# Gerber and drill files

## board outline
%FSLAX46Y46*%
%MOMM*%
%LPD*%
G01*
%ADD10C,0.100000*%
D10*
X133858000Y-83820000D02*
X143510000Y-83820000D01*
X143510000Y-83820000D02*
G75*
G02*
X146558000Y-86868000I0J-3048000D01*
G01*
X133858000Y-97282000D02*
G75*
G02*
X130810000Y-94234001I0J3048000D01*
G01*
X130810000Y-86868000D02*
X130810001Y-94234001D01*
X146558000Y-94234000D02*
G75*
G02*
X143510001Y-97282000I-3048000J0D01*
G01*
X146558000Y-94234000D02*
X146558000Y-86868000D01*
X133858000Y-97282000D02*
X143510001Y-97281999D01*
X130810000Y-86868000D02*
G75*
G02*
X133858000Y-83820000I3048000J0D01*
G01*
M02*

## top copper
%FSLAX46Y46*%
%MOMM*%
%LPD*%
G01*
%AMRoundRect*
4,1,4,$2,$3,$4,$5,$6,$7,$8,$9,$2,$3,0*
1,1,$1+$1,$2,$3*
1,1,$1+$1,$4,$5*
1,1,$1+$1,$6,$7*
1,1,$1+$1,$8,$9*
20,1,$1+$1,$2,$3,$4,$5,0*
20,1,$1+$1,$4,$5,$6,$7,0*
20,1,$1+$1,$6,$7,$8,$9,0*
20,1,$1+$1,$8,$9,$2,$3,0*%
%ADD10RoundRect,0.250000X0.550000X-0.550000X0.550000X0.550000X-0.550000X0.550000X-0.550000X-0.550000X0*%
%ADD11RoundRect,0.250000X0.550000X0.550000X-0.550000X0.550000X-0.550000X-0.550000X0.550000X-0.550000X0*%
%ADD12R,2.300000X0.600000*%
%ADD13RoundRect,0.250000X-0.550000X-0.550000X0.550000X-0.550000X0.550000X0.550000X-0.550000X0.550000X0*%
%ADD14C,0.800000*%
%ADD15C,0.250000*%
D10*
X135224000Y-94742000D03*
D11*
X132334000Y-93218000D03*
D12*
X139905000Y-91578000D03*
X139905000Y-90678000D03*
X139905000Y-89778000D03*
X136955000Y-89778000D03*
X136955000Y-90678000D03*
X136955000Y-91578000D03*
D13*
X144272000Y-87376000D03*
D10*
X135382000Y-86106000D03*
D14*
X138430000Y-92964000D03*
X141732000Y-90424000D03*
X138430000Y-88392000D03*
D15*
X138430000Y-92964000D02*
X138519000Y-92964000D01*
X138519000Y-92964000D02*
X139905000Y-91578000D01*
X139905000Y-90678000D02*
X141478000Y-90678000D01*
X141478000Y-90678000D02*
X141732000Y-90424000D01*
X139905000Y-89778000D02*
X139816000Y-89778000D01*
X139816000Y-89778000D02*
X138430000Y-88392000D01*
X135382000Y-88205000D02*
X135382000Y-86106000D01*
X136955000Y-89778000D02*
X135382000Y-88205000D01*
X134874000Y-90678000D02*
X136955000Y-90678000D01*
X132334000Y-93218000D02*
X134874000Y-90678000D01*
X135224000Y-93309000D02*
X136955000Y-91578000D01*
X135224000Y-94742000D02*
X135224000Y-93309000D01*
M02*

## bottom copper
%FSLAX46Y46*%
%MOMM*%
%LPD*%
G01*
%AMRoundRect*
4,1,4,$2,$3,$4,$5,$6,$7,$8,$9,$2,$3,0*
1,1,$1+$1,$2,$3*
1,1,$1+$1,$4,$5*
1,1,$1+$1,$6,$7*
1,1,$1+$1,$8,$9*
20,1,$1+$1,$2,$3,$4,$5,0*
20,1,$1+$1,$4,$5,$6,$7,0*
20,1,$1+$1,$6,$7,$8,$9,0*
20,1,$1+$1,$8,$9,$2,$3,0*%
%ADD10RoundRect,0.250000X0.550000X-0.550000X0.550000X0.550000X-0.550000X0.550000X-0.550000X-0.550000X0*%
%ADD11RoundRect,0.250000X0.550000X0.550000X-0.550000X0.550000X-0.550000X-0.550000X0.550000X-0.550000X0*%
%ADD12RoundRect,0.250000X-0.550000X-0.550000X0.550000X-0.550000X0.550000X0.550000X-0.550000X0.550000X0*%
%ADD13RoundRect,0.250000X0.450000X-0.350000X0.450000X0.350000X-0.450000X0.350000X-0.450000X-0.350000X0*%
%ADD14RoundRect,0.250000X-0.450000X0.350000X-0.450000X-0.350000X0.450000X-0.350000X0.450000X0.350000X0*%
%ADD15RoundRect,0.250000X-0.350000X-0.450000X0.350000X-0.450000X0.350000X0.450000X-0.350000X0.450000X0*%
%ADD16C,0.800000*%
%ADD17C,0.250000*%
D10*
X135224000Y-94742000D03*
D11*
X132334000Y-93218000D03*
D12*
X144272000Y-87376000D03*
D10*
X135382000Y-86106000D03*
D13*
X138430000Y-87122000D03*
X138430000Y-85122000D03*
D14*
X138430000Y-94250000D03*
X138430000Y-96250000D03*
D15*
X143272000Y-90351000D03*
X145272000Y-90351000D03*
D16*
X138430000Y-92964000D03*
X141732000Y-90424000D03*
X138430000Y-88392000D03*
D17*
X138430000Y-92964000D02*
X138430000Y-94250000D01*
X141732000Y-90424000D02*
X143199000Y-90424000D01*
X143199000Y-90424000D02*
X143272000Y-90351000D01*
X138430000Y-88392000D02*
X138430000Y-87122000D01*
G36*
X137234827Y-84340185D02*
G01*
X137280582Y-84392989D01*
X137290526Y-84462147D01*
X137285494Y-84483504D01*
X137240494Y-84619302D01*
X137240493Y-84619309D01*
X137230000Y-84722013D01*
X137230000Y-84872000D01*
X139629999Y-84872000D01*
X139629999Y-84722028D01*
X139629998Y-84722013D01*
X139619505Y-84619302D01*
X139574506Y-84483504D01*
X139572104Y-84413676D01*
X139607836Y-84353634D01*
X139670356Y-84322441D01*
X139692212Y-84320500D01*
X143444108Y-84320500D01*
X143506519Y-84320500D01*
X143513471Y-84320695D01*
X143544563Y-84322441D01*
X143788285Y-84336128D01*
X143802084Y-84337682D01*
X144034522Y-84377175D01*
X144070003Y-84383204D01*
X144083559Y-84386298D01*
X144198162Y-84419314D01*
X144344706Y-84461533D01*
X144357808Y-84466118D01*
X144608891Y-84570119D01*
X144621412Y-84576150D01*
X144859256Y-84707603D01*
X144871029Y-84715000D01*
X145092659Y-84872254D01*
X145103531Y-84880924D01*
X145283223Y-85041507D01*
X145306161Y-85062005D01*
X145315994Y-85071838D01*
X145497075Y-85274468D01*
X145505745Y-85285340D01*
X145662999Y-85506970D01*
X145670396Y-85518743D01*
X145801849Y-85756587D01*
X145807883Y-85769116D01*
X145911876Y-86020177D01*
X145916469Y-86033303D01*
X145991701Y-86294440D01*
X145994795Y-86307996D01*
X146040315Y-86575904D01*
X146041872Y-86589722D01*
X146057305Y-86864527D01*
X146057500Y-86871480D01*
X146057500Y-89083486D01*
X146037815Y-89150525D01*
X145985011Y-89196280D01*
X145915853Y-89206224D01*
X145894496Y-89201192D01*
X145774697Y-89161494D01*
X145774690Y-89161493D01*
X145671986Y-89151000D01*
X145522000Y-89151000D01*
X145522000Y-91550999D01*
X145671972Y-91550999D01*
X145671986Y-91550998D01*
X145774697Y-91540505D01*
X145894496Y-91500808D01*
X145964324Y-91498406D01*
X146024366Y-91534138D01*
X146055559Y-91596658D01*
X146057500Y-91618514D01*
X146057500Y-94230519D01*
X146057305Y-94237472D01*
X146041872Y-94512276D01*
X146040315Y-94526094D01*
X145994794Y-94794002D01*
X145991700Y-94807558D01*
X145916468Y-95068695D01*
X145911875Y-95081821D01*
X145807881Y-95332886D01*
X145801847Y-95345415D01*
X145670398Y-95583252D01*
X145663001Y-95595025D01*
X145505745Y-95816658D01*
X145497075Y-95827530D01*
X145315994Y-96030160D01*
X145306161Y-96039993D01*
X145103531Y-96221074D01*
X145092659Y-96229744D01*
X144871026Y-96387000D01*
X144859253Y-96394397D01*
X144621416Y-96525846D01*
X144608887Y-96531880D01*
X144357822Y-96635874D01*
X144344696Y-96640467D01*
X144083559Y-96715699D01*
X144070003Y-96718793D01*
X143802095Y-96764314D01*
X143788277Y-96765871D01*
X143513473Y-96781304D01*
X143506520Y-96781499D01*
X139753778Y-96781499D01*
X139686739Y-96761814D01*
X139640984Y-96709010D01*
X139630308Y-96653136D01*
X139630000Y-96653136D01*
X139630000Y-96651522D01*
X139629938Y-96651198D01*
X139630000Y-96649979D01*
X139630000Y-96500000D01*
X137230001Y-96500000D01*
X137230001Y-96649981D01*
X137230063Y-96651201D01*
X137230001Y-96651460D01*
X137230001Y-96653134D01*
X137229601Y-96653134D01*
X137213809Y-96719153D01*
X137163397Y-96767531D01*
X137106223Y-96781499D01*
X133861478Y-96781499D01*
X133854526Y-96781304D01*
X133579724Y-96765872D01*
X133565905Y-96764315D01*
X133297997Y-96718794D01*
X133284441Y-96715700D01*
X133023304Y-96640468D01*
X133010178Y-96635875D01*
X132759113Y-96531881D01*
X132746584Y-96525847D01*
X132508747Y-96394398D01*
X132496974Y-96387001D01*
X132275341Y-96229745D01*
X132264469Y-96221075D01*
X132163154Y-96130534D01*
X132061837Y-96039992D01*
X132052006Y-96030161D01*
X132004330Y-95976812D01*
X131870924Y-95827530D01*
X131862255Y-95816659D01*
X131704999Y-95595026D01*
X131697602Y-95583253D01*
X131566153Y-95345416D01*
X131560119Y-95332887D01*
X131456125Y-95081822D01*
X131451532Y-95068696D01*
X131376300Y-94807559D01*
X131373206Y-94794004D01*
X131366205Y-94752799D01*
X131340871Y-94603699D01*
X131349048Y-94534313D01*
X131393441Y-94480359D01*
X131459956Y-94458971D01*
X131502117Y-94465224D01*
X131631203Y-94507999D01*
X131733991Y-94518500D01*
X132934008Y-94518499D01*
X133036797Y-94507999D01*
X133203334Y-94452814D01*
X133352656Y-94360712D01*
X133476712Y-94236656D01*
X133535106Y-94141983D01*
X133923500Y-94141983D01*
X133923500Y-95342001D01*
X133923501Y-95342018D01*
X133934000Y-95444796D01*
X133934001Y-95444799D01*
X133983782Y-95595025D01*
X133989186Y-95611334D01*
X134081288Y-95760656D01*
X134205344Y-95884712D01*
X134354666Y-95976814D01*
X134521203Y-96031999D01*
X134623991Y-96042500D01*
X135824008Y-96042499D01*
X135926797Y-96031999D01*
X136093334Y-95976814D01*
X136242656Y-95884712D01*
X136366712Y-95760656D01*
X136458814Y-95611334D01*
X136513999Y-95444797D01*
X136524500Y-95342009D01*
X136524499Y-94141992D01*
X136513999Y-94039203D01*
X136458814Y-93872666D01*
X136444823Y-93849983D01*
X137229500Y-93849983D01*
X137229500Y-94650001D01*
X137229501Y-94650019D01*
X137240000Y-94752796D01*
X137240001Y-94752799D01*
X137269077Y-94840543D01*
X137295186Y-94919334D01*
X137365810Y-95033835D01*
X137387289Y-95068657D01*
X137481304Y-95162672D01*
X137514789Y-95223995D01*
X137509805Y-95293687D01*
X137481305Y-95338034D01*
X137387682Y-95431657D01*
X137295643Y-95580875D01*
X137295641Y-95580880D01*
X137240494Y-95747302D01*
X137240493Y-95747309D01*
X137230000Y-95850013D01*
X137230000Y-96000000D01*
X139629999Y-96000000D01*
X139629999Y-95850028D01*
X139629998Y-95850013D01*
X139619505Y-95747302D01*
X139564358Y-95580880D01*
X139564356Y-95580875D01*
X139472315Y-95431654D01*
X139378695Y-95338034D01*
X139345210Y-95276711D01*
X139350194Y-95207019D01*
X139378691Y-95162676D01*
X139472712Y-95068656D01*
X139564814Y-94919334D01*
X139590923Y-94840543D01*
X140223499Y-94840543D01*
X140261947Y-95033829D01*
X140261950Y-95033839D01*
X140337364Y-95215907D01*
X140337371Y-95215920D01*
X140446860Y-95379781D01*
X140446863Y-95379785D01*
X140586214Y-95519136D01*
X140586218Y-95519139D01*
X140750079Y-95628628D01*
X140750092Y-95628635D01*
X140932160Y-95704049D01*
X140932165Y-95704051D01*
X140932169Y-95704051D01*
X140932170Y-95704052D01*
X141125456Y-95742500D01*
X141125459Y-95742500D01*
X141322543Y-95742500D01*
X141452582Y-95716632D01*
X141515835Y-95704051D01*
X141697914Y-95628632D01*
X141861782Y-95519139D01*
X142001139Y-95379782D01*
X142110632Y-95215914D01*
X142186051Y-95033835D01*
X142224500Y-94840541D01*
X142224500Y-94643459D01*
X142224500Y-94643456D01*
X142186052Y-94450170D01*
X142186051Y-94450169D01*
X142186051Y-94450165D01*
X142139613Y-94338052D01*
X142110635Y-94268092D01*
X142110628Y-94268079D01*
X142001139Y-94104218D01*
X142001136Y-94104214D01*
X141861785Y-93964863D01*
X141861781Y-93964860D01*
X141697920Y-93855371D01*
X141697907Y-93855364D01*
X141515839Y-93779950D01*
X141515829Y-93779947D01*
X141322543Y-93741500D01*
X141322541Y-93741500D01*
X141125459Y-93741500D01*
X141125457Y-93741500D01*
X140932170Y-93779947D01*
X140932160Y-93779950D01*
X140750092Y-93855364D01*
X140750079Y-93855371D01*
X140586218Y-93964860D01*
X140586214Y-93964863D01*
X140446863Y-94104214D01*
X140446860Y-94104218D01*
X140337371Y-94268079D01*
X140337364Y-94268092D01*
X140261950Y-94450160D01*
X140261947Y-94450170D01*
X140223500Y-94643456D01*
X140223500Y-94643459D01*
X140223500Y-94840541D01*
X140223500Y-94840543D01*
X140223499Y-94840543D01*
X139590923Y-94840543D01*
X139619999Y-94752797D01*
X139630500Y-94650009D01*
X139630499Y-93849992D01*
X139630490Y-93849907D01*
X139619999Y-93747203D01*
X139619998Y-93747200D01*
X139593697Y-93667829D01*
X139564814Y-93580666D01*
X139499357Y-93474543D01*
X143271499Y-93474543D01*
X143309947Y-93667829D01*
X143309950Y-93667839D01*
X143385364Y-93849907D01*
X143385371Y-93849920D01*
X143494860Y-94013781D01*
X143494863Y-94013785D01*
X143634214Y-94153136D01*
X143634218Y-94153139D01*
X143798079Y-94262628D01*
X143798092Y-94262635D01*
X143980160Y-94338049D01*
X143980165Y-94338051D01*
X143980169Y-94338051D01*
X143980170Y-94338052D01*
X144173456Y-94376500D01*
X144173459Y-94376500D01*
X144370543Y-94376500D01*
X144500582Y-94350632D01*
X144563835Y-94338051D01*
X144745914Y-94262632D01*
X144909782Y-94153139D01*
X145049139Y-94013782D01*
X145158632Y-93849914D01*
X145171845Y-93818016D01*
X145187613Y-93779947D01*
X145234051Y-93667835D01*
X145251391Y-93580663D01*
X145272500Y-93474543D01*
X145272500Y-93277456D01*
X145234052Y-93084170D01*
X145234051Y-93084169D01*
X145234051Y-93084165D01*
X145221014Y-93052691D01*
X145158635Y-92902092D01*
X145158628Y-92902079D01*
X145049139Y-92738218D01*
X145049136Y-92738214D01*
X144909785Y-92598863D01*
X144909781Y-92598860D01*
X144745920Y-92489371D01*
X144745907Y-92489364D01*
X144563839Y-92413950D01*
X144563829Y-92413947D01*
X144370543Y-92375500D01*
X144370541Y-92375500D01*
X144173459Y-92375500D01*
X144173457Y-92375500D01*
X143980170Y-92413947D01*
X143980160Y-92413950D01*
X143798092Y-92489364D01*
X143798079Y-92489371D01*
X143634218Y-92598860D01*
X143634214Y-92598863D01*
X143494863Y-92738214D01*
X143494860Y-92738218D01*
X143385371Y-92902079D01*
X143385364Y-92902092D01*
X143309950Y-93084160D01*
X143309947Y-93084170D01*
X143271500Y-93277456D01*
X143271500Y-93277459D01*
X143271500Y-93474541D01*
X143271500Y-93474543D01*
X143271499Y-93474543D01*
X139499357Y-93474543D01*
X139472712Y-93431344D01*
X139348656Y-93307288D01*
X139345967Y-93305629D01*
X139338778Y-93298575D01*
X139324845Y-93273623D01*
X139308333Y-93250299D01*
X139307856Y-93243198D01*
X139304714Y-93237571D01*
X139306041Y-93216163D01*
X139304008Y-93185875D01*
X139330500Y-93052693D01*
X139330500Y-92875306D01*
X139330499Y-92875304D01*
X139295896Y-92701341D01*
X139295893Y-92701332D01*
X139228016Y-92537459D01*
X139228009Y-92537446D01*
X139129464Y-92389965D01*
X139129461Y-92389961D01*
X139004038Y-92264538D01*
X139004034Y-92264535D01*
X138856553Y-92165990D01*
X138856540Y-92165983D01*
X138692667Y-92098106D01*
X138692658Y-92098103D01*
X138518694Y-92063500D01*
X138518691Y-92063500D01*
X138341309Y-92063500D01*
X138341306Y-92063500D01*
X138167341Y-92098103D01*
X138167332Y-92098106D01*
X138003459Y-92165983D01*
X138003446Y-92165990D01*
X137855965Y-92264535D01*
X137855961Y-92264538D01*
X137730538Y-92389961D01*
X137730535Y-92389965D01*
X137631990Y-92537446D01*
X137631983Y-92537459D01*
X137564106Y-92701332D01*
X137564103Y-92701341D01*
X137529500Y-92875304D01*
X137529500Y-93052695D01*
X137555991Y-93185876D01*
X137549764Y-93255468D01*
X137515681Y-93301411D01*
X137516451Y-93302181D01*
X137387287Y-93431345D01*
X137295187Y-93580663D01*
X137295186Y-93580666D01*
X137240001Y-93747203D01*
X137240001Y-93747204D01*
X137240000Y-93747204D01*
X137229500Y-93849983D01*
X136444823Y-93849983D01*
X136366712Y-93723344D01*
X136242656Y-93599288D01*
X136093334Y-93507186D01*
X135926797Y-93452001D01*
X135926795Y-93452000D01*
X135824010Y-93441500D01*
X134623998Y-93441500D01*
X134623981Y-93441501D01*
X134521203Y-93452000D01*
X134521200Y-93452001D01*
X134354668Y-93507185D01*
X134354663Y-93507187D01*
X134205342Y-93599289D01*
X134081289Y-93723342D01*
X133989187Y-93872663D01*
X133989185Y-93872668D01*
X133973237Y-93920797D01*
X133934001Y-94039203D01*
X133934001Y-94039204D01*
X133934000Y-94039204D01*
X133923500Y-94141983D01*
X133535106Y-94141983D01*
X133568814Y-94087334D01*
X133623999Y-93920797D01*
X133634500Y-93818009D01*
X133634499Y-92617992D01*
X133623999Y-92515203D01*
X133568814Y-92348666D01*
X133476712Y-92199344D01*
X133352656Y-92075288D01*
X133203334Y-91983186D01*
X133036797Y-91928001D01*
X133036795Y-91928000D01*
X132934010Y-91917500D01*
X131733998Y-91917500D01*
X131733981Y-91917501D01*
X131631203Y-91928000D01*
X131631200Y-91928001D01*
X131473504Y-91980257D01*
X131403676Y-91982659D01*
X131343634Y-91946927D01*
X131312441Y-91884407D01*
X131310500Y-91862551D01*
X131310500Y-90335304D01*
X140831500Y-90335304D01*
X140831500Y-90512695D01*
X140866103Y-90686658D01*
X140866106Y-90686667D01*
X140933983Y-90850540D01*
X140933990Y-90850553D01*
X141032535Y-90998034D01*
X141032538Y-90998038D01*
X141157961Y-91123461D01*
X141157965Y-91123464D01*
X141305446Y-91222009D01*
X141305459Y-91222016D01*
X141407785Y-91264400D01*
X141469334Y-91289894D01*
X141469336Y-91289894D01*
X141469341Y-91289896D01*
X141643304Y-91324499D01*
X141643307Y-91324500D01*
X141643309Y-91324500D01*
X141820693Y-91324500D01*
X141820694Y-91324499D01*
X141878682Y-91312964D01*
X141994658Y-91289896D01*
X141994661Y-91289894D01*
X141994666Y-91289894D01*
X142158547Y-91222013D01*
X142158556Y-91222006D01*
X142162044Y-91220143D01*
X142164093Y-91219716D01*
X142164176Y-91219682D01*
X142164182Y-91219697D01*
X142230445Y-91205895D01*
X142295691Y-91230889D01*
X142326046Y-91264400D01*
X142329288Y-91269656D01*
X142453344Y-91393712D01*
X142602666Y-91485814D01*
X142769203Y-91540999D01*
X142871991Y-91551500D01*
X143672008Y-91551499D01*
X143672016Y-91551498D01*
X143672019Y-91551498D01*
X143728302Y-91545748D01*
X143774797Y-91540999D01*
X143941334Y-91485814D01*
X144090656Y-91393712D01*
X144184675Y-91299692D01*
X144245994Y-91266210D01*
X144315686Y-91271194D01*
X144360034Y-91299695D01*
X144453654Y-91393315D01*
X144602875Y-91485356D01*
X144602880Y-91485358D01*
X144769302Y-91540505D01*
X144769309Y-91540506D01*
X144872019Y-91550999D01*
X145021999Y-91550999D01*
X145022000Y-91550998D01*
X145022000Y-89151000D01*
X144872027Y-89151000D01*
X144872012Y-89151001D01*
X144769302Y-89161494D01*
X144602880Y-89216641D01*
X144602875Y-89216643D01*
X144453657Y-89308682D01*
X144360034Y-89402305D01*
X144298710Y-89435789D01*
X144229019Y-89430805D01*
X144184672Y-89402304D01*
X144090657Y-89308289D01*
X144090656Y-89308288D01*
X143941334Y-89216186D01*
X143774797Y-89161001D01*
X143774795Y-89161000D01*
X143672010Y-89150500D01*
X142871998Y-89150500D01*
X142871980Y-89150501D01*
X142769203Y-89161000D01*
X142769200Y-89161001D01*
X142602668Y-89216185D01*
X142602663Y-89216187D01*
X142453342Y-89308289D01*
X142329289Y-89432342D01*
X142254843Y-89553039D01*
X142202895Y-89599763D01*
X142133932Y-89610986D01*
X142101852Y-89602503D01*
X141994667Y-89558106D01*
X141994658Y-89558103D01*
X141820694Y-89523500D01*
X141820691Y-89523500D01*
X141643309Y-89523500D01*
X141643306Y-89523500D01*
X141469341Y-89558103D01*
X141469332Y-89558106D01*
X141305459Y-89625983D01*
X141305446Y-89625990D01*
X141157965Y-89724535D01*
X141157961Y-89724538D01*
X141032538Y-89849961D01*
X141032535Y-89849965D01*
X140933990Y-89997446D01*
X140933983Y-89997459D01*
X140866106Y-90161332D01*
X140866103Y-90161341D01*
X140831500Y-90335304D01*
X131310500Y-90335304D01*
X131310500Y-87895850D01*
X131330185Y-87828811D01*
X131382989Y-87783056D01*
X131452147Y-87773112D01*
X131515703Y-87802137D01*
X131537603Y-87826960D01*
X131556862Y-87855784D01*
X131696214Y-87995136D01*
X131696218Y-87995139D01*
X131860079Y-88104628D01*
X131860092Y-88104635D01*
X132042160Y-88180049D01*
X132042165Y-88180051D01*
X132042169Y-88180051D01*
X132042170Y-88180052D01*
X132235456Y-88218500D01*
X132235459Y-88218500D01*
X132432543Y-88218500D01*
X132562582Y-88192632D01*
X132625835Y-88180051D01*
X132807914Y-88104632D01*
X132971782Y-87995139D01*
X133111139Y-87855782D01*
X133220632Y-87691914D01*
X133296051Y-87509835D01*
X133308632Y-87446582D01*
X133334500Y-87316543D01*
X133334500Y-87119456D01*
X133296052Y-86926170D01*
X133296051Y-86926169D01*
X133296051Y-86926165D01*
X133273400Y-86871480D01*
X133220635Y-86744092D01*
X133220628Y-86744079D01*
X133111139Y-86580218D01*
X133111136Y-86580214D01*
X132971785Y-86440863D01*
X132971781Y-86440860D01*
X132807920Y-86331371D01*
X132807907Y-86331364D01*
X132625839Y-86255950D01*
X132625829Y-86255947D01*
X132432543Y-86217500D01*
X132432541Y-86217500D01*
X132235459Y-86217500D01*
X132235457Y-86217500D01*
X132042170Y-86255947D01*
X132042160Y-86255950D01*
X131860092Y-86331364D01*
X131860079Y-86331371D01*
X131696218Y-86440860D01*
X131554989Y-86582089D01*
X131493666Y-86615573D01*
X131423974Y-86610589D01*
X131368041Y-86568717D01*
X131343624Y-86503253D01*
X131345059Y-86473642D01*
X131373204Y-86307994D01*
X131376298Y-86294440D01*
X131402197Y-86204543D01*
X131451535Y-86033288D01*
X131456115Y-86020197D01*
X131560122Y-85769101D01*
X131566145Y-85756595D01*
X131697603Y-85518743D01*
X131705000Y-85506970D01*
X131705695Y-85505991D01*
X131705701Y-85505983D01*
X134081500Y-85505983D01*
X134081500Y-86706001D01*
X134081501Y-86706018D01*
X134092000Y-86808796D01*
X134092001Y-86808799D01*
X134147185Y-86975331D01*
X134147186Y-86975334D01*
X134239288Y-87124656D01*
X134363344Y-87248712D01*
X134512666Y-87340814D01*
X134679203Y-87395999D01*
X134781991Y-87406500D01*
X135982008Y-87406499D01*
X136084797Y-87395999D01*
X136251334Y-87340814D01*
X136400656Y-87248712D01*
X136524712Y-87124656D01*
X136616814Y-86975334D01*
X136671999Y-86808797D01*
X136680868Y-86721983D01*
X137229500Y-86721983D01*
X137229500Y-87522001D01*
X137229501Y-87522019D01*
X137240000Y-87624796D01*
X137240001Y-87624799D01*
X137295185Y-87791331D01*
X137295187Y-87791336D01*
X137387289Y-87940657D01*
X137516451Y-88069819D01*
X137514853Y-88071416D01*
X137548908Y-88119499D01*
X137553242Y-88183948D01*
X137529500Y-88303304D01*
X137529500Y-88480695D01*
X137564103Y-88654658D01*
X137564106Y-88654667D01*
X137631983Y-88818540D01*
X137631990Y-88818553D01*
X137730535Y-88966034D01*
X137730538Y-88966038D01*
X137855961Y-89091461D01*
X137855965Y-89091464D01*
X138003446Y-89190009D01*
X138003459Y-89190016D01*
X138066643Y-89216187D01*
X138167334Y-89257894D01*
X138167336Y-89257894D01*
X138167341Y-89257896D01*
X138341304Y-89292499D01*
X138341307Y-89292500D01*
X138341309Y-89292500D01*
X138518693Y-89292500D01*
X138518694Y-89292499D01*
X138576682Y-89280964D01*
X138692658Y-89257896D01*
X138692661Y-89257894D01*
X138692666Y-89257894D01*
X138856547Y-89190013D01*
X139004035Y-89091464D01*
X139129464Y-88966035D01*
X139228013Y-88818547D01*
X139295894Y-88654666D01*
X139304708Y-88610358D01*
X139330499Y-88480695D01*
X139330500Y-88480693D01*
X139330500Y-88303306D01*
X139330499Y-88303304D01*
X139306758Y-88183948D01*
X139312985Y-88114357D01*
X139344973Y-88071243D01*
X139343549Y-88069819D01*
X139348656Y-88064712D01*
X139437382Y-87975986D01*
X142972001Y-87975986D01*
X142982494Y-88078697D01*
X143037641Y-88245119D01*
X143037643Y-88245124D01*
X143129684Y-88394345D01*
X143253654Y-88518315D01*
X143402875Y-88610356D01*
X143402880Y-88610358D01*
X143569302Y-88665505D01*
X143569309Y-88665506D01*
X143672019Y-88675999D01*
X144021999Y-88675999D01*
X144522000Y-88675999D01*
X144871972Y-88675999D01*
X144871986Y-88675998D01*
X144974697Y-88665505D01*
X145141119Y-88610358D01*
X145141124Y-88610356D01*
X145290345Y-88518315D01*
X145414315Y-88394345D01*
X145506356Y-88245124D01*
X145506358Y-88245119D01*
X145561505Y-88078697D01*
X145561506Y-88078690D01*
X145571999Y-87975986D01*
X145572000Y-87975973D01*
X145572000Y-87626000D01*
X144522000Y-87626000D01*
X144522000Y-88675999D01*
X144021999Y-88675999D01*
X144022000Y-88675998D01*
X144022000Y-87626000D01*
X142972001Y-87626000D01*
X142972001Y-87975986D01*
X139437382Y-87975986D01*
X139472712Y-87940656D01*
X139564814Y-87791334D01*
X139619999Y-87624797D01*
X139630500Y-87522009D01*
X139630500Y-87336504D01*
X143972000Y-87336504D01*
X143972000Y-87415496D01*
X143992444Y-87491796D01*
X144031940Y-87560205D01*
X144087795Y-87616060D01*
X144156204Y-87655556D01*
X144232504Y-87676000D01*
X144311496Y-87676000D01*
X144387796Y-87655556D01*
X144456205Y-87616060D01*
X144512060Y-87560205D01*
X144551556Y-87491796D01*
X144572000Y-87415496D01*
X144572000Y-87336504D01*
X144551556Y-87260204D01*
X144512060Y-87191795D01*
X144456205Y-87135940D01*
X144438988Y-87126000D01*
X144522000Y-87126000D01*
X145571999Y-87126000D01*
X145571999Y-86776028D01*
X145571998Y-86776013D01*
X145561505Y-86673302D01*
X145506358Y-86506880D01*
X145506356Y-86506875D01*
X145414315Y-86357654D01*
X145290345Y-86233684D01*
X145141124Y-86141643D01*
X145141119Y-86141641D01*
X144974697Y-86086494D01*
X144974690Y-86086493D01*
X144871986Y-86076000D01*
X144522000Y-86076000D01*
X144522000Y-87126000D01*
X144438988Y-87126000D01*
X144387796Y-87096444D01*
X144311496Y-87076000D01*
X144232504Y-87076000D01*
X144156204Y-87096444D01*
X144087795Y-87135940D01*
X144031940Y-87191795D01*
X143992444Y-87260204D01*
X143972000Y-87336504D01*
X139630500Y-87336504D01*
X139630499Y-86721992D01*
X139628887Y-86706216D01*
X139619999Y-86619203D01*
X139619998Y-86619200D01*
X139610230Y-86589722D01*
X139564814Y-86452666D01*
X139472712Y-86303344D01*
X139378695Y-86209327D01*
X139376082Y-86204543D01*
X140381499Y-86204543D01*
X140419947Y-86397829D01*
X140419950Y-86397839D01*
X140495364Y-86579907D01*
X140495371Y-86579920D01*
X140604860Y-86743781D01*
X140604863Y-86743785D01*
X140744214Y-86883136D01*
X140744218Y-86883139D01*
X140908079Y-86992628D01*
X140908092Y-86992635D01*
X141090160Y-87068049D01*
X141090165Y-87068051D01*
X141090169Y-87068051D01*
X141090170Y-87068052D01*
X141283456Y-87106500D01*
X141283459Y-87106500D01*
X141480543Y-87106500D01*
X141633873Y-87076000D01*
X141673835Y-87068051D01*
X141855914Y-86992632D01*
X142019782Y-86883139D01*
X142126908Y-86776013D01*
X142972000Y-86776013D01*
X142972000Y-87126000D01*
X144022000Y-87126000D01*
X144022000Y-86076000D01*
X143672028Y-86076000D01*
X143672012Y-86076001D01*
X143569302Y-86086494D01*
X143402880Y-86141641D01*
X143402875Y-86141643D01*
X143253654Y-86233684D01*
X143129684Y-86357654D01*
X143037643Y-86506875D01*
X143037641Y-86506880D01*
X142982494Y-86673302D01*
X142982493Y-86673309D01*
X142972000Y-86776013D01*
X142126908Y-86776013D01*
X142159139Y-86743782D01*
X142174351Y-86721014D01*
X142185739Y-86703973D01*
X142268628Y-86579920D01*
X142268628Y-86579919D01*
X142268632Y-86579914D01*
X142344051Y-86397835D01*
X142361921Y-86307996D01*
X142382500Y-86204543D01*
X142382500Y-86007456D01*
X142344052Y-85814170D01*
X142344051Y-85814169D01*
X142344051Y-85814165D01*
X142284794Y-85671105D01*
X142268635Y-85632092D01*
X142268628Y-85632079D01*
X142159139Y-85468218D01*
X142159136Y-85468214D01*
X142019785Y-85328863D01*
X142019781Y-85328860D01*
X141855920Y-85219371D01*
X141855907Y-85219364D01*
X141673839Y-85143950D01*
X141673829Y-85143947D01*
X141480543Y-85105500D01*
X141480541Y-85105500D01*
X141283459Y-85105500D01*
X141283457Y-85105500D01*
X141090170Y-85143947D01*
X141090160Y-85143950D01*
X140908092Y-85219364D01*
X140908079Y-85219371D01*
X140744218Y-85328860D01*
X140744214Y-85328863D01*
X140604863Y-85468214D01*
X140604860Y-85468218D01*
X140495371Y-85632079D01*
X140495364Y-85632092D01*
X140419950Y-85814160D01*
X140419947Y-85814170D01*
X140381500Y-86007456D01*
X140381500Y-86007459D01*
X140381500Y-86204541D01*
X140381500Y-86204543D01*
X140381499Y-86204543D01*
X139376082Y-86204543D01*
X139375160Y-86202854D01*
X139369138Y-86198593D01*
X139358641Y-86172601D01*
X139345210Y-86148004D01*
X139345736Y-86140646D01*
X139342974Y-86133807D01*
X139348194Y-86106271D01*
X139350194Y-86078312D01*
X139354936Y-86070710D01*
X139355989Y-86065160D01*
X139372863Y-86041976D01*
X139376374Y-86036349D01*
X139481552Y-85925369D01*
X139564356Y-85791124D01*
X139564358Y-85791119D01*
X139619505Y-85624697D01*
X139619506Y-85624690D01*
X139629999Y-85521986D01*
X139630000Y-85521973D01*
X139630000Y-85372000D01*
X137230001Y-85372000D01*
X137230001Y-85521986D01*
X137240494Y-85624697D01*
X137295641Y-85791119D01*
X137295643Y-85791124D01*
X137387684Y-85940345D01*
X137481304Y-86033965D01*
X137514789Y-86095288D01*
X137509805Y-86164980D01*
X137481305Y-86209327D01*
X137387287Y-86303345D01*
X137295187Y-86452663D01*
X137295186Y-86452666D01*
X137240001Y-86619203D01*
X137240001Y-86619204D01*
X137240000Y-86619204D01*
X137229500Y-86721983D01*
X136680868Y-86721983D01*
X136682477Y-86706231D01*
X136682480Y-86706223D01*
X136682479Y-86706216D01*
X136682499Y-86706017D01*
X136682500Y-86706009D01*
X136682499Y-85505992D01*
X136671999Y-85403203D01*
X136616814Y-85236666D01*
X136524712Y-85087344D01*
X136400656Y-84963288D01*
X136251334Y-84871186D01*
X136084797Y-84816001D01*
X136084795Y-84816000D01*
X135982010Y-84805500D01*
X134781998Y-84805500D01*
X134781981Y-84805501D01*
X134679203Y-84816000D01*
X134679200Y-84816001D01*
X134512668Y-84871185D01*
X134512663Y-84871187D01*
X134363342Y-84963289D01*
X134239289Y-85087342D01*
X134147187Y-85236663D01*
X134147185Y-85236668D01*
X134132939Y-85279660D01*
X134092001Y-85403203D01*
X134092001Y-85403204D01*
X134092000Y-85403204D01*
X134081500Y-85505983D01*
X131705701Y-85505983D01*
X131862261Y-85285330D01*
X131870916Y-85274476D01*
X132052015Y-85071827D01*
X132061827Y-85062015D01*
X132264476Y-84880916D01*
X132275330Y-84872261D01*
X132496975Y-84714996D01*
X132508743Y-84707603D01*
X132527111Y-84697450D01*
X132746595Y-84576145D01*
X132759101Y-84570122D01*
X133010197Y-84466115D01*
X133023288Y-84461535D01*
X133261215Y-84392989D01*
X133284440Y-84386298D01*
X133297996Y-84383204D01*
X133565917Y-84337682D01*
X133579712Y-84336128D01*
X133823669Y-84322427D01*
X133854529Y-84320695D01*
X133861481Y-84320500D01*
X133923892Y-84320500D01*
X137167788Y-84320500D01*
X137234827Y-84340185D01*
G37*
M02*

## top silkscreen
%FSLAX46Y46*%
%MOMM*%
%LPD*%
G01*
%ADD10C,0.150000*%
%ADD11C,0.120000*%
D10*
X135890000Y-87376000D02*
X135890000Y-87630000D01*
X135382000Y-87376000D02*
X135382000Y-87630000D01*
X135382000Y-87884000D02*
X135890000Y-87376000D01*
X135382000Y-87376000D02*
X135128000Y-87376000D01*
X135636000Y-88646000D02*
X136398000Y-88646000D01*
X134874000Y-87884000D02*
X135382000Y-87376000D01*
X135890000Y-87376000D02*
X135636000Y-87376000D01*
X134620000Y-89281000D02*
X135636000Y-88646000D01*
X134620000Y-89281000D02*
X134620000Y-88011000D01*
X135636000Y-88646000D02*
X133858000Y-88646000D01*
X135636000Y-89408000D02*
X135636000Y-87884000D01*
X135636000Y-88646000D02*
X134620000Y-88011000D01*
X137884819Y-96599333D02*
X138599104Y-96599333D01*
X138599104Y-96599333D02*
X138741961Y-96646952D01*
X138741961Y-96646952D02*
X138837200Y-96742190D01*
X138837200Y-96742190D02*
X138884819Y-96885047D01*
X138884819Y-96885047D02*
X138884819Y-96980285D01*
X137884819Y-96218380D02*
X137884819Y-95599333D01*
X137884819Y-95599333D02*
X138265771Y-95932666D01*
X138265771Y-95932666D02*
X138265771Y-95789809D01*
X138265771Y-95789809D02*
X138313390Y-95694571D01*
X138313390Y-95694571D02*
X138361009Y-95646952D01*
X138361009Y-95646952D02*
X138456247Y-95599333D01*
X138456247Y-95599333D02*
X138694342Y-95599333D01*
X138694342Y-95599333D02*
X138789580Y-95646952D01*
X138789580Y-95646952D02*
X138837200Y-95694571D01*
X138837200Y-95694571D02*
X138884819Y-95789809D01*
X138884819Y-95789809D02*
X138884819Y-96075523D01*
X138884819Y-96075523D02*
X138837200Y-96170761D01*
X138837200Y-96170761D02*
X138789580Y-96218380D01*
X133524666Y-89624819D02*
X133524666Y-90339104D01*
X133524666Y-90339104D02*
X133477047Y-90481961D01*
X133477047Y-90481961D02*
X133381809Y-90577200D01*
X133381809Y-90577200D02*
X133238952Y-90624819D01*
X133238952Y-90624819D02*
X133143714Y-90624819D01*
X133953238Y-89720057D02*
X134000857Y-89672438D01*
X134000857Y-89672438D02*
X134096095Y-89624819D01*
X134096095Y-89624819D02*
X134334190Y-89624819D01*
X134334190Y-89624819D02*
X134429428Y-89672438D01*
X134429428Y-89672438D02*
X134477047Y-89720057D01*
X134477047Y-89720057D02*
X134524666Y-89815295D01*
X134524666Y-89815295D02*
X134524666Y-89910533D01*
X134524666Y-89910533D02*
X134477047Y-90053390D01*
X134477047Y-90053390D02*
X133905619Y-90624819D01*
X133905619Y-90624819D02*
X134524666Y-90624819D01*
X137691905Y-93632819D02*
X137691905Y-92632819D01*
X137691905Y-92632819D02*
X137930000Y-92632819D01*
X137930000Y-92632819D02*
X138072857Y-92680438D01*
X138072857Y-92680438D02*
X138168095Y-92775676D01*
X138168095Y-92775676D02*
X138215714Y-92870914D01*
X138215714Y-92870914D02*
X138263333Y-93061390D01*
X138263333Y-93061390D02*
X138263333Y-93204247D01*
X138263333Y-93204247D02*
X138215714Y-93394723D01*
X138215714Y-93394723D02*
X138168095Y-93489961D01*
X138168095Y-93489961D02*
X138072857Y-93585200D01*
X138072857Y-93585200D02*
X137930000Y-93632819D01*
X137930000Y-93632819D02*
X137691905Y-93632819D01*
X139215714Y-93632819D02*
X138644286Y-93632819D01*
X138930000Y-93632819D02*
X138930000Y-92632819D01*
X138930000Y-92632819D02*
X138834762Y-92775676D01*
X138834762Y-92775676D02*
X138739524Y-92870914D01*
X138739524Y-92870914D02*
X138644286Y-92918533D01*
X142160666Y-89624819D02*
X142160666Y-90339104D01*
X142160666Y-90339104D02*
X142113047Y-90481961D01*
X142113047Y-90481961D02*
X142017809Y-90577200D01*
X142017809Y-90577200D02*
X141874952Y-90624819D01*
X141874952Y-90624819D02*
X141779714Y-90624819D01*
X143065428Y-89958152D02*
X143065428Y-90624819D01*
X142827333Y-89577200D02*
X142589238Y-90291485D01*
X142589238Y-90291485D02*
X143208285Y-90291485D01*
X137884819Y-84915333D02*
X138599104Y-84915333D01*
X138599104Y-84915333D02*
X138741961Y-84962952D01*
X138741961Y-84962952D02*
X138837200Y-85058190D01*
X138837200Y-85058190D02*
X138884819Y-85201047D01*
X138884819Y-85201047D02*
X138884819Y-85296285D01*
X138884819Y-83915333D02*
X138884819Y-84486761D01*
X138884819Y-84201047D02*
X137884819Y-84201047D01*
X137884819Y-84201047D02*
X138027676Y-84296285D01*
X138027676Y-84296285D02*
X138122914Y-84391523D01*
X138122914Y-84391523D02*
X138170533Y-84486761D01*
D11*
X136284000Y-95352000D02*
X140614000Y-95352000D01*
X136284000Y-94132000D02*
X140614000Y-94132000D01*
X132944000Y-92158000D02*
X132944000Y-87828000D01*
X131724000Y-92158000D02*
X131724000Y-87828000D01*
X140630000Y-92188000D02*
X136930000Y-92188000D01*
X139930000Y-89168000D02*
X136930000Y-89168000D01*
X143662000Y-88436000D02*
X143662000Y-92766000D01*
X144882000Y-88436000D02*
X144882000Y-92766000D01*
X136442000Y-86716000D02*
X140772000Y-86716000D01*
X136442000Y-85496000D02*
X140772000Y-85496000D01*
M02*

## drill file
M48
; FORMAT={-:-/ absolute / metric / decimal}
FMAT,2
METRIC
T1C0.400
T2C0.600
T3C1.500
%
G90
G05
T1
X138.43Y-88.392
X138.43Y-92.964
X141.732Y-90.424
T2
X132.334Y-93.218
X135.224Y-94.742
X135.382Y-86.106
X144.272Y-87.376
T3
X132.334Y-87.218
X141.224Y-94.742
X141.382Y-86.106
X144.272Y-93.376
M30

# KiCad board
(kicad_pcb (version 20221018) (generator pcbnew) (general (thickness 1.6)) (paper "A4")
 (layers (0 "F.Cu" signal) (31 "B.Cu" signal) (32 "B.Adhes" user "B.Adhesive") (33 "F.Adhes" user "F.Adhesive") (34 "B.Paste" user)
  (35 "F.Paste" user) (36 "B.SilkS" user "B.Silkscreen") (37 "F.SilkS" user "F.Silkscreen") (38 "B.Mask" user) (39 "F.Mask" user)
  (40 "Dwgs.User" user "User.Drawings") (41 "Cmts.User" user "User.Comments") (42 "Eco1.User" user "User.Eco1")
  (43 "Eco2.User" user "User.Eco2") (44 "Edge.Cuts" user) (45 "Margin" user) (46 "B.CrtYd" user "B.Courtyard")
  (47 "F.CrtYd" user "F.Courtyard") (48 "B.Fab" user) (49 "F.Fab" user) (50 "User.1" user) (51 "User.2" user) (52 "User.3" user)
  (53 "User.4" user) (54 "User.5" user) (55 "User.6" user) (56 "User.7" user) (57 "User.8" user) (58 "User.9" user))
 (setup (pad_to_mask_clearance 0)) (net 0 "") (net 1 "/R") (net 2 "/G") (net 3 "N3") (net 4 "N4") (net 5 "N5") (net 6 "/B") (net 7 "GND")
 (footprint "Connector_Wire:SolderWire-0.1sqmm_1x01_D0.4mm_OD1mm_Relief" (layer "F.Cu") (at 135.224 94.742 90)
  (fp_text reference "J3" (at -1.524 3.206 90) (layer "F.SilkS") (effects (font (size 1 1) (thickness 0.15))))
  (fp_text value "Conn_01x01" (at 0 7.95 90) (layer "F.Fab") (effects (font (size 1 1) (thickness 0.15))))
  (fp_line (start -0.61 1.06) (end -0.61 5.39) (stroke (width 0.12) (type solid)) (layer "F.SilkS"))
  (fp_line (start 0.61 1.06) (end 0.61 5.39) (stroke (width 0.12) (type solid)) (layer "F.SilkS"))
  (pad "" np_thru_hole circle (at 0 6 90) (size 1.5 1.5) (drill 1.5) (layers "*.Cu" "*.Mask"))
  (pad "1" thru_hole roundrect (at 0 0 90) (size 1.6 1.6) (drill 0.6) (layers "*.Cu" "*.Mask") (roundrect_rratio 0.15625) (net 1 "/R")))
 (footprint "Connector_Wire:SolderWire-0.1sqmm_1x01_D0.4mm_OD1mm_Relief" (layer "F.Cu") (at 132.334 93.218 180)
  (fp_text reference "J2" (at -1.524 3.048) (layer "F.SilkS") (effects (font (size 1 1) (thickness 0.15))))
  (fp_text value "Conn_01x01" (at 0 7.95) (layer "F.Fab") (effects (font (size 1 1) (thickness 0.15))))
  (fp_line (start -0.61 1.06) (end -0.61 5.39) (stroke (width 0.12) (type solid)) (layer "F.SilkS"))
  (fp_line (start 0.61 1.06) (end 0.61 5.39) (stroke (width 0.12) (type solid)) (layer "F.SilkS"))
  (pad "" np_thru_hole circle (at 0 6 180) (size 1.5 1.5) (drill 1.5) (layers "*.Cu" "*.Mask"))
  (pad "1" thru_hole roundrect (at 0 0 180) (size 1.6 1.6) (drill 0.6) (layers "*.Cu" "*.Mask") (roundrect_rratio 0.15625) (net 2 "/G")))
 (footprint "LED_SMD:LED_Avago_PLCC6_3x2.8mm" (layer "F.Cu") (at 138.43 90.678 180)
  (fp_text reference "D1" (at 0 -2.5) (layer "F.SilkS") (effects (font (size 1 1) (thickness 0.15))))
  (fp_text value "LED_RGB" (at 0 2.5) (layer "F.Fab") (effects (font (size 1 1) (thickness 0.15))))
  (fp_line (start -2.2 -1.51) (end 1.5 -1.51) (stroke (width 0.12) (type solid)) (layer "F.SilkS"))
  (fp_line (start -1.5 1.51) (end 1.5 1.51) (stroke (width 0.12) (type solid)) (layer "F.SilkS"))
  (pad "1" smd rect (at -1.475 -0.9 180) (size 2.3 0.6) (layers "F.Cu" "F.Paste" "F.Mask") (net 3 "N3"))
  (pad "2" smd rect (at -1.475 0 180) (size 2.3 0.6) (layers "F.Cu" "F.Paste" "F.Mask") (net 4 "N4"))
  (pad "3" smd rect (at -1.475 0.9 180) (size 2.3 0.6) (layers "F.Cu" "F.Paste" "F.Mask") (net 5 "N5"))
  (pad "4" smd rect (at 1.475 0.9 180) (size 2.3 0.6) (layers "F.Cu" "F.Paste" "F.Mask") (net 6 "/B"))
  (pad "5" smd rect (at 1.475 0 180) (size 2.3 0.6) (layers "F.Cu" "F.Paste" "F.Mask") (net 2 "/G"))
  (pad "6" smd rect (at 1.475 -0.9 180) (size 2.3 0.6) (layers "F.Cu" "F.Paste" "F.Mask") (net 1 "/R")))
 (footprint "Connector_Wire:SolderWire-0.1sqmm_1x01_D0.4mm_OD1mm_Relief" (layer "F.Cu") (at 144.272 87.376)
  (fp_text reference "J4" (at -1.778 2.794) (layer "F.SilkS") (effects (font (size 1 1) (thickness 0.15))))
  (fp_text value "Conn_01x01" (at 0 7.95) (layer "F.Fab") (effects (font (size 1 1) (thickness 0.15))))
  (fp_line (start -0.61 1.06) (end -0.61 5.39) (stroke (width 0.12) (type solid)) (layer "F.SilkS"))
  (fp_line (start 0.61 1.06) (end 0.61 5.39) (stroke (width 0.12) (type solid)) (layer "F.SilkS"))
  (pad "" np_thru_hole circle (at 0 6) (size 1.5 1.5) (drill 1.5) (layers "*.Cu" "*.Mask"))
  (pad "1" thru_hole roundrect (at 0 0) (size 1.6 1.6) (drill 0.6) (layers "*.Cu" "*.Mask") (roundrect_rratio 0.15625) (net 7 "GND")))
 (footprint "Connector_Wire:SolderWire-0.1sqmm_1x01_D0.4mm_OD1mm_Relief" (layer "F.Cu") (at 135.382 86.106 90)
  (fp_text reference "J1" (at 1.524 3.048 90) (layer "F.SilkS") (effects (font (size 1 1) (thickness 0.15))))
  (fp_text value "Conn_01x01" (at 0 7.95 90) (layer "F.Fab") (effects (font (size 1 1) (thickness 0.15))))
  (fp_line (start -0.61 1.06) (end -0.61 5.39) (stroke (width 0.12) (type solid)) (layer "F.SilkS"))
  (fp_line (start 0.61 1.06) (end 0.61 5.39) (stroke (width 0.12) (type solid)) (layer "F.SilkS"))
  (pad "" np_thru_hole circle (at 0 6 90) (size 1.5 1.5) (drill 1.5) (layers "*.Cu" "*.Mask"))
  (pad "1" thru_hole roundrect (at 0 0 90) (size 1.6 1.6) (drill 0.6) (layers "*.Cu" "*.Mask") (roundrect_rratio 0.15625) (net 6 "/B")))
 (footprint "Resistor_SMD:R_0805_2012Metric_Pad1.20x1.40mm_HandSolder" (layer "B.Cu") (at 138.43 86.122 90)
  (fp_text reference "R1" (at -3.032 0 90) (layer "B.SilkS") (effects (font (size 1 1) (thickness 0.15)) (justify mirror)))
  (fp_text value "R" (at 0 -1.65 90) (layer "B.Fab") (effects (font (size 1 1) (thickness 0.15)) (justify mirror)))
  (pad "1" smd roundrect (at -1 0 90) (size 1.2 1.4) (layers "B.Cu" "B.Paste" "B.Mask") (roundrect_rratio 0.208333) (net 5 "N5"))
  (pad "2" smd roundrect (at 1 0 90) (size 1.2 1.4) (layers "B.Cu" "B.Paste" "B.Mask") (roundrect_rratio 0.208333) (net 7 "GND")))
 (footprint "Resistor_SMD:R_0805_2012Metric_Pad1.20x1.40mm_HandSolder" (layer "B.Cu") (at 138.43 95.25 -90)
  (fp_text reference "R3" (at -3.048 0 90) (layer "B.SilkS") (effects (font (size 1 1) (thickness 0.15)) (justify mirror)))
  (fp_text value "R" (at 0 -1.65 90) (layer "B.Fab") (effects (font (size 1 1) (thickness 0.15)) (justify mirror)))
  (pad "1" smd roundrect (at -1 0 270) (size 1.2 1.4) (layers "B.Cu" "B.Paste" "B.Mask") (roundrect_rratio 0.208333) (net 3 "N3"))
  (pad "2" smd roundrect (at 1 0 270) (size 1.2 1.4) (layers "B.Cu" "B.Paste" "B.Mask") (roundrect_rratio 0.208333) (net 7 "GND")))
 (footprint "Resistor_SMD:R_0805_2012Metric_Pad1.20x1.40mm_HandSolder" (layer "B.Cu") (at 144.272 90.351)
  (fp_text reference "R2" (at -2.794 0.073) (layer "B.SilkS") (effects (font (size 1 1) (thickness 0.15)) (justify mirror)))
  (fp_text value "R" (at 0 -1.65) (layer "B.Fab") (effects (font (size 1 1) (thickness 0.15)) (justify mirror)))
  (pad "1" smd roundrect (at -1 0) (size 1.2 1.4) (layers "B.Cu" "B.Paste" "B.Mask") (roundrect_rratio 0.208333) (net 4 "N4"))
  (pad "2" smd roundrect (at 1 0) (size 1.2 1.4) (layers "B.Cu" "B.Paste" "B.Mask") (roundrect_rratio 0.208333) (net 7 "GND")))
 (gr_line (start 135.89 87.376) (end 135.89 87.63) (stroke (width 0.15) (type default)) (layer "F.SilkS"))
 (gr_line (start 135.382 87.376) (end 135.382 87.63) (stroke (width 0.15) (type default)) (layer "F.SilkS"))
 (gr_line (start 135.382 87.884) (end 135.89 87.376) (stroke (width 0.15) (type default)) (layer "F.SilkS"))
 (gr_line (start 135.382 87.376) (end 135.128 87.376) (stroke (width 0.15) (type default)) (layer "F.SilkS"))
 (gr_line (start 135.636 88.646) (end 136.398 88.646) (stroke (width 0.15) (type default)) (layer "F.SilkS"))
 (gr_line (start 134.874 87.884) (end 135.382 87.376) (stroke (width 0.15) (type default)) (layer "F.SilkS"))
 (gr_line (start 135.89 87.376) (end 135.636 87.376) (stroke (width 0.15) (type default)) (layer "F.SilkS"))
 (gr_line (start 134.62 89.281) (end 135.636 88.646) (stroke (width 0.15) (type default)) (layer "F.SilkS"))
 (gr_line (start 134.62 89.281) (end 134.62 88.011) (stroke (width 0.15) (type default)) (layer "F.SilkS"))
 (gr_line (start 135.636 88.646) (end 133.858 88.646) (stroke (width 0.15) (type default)) (layer "F.SilkS"))
 (gr_line (start 135.636 89.408) (end 135.636 87.884) (stroke (width 0.15) (type default)) (layer "F.SilkS"))
 (gr_line (start 135.636 88.646) (end 134.62 88.011) (stroke (width 0.15) (type default)) (layer "F.SilkS"))
 (gr_line (start 133.858 83.82) (end 143.51 83.82) (stroke (width 0.1) (type default)) (layer "Edge.Cuts"))
 (gr_arc (start 143.51 83.82) (mid 145.665261 84.712739) (end 146.558 86.868) (stroke (width 0.1) (type default)) (layer "Edge.Cuts"))
 (gr_arc (start 133.858 97.282) (mid 131.70274 96.389261) (end 130.810001 94.234001) (stroke (width 0.1) (type default)) (layer "Edge.Cuts"))
 (gr_line (start 130.81 86.868) (end 130.810001 94.234001) (stroke (width 0.1) (type default)) (layer "Edge.Cuts"))
 (gr_arc (start 146.558 94.234) (mid 145.665261 96.38926) (end 143.510001 97.281999) (stroke (width 0.1) (type default)) (layer "Edge.Cuts"))
 (gr_line (start 146.558 94.234) (end 146.558 86.868) (stroke (width 0.1) (type default)) (layer "Edge.Cuts"))
 (gr_line (start 133.858 97.282) (end 143.510001 97.281999) (stroke (width 0.1) (type default)) (layer "Edge.Cuts"))
 (gr_arc (start 130.81 86.868) (mid 131.702739 84.712739) (end 133.858 83.82) (stroke (width 0.1) (type default)) (layer "Edge.Cuts"))
 (segment (start 138.43 92.964) (end 138.519 92.964) (width 0.25) (layer "F.Cu") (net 3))
 (segment (start 138.519 92.964) (end 139.905 91.578) (width 0.25) (layer "F.Cu") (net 3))
 (via (at 138.43 92.964) (size 0.8) (drill 0.4) (layers "F.Cu" "B.Cu") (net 3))
 (segment (start 138.43 92.964) (end 138.43 94.25) (width 0.25) (layer "B.Cu") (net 3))
 (segment (start 139.905 90.678) (end 141.478 90.678) (width 0.25) (layer "F.Cu") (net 4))
 (segment (start 141.478 90.678) (end 141.732 90.424) (width 0.25) (layer "F.Cu") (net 4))
 (via (at 141.732 90.424) (size 0.8) (drill 0.4) (layers "F.Cu" "B.Cu") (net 4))
 (segment (start 141.732 90.424) (end 143.199 90.424) (width 0.25) (layer "B.Cu") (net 4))
 (segment (start 143.199 90.424) (end 143.272 90.351) (width 0.25) (layer "B.Cu") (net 4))
 (segment (start 139.905 89.778) (end 139.816 89.778) (width 0.25) (layer "F.Cu") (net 5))
 (segment (start 139.816 89.778) (end 138.43 88.392) (width 0.25) (layer "F.Cu") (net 5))
 (via (at 138.43 88.392) (size 0.8) (drill 0.4) (layers "F.Cu" "B.Cu") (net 5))
 (segment (start 138.43 88.392) (end 138.43 87.122) (width 0.25) (layer "B.Cu") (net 5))
 (segment (start 135.382 88.205) (end 135.382 86.106) (width 0.25) (layer "F.Cu") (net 6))
 (segment (start 136.955 89.778) (end 135.382 88.205) (width 0.25) (layer "F.Cu") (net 6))
 (segment (start 134.874 90.678) (end 136.955 90.678) (width 0.25) (layer "F.Cu") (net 2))
 (segment (start 132.334 93.218) (end 134.874 90.678) (width 0.25) (layer "F.Cu") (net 2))
 (segment (start 135.224 93.309) (end 136.955 91.578) (width 0.25) (layer "F.Cu") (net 1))
 (segment (start 135.224 94.742) (end 135.224 93.309) (width 0.25) (layer "F.Cu") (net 1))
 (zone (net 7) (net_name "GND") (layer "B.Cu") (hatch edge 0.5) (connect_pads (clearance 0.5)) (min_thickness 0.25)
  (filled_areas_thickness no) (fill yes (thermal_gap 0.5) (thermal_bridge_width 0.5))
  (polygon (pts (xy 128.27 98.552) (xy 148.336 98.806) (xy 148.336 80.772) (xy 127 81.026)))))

